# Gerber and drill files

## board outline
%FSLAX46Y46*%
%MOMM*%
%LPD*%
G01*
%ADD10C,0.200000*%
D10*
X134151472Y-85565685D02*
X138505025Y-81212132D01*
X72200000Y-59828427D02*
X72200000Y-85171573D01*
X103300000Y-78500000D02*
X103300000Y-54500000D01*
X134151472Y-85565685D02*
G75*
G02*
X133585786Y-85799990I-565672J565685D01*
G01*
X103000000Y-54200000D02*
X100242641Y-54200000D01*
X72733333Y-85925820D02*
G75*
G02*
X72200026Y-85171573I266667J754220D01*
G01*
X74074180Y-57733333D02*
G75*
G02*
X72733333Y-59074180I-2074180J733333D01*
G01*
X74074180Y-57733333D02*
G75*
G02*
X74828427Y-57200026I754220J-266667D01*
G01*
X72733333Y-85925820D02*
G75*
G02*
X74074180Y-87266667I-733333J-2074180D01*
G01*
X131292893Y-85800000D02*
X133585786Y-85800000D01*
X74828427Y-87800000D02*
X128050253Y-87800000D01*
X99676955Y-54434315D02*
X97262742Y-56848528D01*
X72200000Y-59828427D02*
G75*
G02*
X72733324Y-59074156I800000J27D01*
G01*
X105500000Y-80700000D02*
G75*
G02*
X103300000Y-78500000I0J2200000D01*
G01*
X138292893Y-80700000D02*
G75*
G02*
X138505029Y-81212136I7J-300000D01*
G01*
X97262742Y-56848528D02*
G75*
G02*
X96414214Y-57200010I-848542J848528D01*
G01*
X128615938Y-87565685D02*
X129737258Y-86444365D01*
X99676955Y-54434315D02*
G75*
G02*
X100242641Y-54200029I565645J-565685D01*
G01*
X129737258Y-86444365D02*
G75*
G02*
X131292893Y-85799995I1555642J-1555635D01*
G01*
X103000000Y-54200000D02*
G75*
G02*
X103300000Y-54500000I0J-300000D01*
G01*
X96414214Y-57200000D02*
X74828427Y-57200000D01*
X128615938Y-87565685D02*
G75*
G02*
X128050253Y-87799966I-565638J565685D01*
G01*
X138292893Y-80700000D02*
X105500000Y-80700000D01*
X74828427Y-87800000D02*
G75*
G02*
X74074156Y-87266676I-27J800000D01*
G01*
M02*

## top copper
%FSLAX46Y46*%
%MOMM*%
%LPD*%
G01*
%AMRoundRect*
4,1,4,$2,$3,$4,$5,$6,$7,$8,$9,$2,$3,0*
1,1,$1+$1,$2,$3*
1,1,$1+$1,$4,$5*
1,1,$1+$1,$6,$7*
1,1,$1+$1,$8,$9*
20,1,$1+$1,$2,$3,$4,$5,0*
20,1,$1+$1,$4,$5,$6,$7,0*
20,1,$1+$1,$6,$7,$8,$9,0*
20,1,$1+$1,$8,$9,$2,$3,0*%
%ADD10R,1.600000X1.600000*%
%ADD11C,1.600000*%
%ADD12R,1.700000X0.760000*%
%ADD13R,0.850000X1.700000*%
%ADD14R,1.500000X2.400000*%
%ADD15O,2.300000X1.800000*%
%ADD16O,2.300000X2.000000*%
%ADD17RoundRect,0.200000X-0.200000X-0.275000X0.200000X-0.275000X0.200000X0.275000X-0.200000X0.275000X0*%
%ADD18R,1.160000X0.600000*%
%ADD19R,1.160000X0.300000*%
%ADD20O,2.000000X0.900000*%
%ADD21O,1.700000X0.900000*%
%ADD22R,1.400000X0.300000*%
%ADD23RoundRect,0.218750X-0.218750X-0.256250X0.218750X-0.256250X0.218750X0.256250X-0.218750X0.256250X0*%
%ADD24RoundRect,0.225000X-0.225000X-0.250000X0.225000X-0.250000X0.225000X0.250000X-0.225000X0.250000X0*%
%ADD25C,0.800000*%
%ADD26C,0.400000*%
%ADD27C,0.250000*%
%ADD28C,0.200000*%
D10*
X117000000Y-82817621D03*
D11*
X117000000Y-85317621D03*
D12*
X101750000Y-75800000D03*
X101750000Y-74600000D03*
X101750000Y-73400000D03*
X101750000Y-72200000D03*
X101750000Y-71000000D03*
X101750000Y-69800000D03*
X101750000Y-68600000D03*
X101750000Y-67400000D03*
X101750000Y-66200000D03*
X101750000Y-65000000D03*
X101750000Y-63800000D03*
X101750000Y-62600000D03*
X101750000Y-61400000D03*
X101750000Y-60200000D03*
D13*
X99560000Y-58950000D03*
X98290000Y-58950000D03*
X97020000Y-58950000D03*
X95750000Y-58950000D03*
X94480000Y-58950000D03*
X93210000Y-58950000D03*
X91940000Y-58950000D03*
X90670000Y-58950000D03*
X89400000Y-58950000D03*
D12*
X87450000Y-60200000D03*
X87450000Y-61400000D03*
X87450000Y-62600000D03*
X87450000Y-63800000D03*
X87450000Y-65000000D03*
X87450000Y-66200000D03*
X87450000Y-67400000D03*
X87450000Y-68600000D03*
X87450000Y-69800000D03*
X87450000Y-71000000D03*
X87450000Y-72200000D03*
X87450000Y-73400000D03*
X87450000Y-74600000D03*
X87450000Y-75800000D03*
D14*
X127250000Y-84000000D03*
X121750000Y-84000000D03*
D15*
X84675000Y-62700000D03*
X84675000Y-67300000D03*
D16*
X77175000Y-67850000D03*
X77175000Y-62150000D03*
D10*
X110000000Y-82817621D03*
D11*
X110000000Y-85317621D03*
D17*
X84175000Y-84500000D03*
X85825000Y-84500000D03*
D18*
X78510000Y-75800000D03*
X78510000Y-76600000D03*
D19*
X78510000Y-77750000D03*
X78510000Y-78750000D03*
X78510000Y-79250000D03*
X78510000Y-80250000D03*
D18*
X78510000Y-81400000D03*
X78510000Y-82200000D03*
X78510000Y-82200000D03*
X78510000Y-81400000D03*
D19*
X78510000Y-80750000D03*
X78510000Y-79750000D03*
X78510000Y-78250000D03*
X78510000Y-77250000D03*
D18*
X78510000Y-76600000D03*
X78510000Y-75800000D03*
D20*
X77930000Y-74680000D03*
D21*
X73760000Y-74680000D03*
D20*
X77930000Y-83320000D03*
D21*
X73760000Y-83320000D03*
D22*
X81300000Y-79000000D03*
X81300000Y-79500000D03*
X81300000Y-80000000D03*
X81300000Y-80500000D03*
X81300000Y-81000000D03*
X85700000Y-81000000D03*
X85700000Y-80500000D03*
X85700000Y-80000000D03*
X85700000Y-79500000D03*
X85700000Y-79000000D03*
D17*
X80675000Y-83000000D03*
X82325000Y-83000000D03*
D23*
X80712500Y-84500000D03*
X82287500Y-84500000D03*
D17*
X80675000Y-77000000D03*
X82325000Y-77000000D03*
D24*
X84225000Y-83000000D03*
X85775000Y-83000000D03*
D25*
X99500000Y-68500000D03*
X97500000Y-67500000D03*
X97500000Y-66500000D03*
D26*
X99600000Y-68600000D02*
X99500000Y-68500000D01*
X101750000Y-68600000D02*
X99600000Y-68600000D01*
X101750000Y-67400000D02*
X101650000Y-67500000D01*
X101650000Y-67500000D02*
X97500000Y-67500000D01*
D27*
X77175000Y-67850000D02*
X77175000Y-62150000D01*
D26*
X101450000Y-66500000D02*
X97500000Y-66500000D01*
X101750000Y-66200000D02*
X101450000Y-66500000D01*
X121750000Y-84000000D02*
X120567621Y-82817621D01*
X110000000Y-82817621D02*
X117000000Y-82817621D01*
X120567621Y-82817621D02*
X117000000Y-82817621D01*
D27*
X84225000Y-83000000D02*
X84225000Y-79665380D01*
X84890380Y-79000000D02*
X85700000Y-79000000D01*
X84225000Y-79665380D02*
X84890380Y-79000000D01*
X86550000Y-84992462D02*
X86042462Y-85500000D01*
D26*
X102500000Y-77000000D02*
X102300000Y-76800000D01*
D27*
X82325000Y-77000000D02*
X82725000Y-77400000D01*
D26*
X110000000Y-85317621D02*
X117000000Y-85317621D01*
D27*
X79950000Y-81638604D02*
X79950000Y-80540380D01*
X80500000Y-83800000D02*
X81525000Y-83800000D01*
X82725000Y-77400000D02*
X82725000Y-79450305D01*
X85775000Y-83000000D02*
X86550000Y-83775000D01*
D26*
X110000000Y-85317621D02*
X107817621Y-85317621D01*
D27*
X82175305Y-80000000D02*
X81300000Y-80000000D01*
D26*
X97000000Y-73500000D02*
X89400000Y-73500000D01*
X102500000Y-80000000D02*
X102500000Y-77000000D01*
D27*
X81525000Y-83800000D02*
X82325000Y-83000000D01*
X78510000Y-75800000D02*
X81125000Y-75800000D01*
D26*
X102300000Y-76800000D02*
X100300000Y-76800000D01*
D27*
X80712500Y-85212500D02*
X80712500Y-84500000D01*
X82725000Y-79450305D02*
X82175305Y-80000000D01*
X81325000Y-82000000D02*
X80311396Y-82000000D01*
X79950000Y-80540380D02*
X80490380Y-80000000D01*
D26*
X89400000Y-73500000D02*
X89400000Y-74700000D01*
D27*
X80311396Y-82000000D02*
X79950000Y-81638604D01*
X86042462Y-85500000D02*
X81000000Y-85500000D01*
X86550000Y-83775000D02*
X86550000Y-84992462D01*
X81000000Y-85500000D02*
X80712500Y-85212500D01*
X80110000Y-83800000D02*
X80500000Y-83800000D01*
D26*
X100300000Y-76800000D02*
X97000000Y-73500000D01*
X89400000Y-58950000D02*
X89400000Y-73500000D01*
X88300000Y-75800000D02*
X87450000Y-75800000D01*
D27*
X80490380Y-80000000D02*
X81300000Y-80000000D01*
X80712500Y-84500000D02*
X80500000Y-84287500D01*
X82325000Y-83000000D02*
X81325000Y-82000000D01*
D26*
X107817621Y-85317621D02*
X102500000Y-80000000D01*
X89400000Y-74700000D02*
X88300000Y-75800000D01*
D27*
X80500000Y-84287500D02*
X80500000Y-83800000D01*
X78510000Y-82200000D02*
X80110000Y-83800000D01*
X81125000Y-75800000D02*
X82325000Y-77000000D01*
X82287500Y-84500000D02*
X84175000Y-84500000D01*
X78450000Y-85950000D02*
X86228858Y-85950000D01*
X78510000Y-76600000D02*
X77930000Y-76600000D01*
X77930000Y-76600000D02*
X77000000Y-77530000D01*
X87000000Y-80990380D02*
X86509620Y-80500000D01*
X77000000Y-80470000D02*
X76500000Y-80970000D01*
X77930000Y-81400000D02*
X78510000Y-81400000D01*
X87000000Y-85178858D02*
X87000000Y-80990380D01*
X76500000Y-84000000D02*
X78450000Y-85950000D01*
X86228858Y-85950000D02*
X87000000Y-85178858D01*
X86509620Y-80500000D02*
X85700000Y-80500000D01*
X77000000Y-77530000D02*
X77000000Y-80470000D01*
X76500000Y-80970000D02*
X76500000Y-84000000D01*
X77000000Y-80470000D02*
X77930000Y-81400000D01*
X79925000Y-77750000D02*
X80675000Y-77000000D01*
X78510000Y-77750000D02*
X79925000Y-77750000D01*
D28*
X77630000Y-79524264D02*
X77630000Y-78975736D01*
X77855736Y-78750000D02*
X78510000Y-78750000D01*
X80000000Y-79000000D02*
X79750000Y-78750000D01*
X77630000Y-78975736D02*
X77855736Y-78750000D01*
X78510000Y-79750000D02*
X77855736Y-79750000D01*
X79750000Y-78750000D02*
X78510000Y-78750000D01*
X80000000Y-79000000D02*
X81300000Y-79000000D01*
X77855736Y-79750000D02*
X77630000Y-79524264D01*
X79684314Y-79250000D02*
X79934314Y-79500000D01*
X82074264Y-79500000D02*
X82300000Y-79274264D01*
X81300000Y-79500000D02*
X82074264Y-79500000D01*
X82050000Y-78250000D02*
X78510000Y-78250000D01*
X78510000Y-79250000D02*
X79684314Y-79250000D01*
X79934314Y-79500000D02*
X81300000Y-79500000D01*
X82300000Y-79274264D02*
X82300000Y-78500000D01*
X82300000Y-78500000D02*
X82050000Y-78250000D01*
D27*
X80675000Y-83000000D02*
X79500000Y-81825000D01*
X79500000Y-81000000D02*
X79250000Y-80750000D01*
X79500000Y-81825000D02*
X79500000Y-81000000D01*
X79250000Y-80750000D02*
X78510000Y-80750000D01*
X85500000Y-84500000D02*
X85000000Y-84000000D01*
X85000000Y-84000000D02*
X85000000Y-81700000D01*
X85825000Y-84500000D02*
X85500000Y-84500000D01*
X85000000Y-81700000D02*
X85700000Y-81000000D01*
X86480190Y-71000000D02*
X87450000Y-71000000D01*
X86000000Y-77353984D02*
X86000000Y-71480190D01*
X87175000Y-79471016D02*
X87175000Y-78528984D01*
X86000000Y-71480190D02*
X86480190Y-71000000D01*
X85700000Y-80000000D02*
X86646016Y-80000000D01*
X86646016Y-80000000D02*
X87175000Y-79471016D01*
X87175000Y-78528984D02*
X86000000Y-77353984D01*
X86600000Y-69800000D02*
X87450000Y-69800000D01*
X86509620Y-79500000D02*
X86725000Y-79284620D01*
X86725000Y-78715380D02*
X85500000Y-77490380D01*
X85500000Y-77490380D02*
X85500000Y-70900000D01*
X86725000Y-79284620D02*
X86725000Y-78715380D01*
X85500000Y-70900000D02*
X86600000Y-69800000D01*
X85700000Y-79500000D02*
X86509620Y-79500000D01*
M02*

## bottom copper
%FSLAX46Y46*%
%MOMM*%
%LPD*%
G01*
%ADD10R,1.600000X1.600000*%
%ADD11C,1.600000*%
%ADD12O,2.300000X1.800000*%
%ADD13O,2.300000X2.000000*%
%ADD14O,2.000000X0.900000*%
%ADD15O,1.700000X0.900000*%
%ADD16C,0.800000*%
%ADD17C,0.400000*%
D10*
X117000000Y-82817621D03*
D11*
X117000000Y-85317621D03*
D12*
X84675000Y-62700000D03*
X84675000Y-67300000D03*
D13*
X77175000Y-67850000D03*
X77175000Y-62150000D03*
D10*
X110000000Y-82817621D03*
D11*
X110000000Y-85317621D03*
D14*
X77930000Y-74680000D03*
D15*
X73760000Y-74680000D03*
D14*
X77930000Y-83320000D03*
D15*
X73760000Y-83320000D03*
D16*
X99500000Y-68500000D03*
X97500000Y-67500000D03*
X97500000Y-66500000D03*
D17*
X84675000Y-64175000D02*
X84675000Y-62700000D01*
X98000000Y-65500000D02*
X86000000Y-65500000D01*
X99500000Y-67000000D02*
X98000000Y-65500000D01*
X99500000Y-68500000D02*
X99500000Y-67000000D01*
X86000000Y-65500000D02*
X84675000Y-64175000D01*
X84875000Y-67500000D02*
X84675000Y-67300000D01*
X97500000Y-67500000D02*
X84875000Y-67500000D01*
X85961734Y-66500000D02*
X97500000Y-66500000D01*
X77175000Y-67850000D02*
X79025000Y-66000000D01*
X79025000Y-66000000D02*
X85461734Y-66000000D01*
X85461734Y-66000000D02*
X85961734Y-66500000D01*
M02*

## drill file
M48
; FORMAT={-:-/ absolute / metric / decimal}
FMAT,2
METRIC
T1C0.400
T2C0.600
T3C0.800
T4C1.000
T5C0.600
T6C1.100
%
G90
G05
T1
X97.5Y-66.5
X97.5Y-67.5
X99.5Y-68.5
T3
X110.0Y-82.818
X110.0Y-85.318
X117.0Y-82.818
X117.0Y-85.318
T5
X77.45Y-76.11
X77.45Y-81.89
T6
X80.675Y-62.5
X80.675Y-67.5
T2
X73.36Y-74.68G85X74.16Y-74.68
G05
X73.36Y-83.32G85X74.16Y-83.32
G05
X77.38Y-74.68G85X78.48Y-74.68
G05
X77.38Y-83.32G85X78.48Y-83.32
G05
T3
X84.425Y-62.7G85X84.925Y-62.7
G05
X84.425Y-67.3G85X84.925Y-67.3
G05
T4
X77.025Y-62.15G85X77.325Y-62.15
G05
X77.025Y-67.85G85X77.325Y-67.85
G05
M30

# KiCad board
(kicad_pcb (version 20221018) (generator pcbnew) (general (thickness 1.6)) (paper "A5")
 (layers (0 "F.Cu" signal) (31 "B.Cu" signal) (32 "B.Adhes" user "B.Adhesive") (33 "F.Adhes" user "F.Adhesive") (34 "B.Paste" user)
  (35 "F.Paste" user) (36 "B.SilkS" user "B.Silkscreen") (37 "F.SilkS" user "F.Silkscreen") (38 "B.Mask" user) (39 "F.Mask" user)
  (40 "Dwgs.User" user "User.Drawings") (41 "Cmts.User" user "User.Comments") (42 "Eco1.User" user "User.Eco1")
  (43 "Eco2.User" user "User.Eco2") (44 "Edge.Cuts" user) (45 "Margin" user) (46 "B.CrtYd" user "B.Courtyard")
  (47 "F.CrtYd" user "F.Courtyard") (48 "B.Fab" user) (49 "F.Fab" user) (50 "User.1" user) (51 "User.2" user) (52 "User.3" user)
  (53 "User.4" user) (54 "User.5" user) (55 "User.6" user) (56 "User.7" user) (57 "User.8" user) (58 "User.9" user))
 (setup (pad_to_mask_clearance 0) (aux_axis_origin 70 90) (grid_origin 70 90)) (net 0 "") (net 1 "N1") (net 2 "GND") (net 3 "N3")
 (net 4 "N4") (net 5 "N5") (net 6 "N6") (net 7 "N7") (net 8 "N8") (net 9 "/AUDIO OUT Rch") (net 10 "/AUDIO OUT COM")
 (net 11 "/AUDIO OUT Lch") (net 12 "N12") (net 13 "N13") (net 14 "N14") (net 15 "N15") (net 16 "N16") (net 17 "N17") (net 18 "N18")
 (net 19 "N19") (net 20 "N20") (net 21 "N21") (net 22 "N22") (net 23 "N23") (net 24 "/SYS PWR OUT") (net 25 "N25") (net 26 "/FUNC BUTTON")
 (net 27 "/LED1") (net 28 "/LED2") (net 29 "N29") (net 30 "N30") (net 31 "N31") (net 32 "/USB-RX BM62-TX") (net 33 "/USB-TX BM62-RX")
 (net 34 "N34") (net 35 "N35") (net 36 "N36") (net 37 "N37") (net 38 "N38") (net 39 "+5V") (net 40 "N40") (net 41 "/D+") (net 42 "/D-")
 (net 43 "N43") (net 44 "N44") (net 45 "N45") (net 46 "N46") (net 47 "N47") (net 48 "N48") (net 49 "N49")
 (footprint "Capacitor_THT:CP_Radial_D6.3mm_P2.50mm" (layer "F.Cu") (at 117 82.817621 -90)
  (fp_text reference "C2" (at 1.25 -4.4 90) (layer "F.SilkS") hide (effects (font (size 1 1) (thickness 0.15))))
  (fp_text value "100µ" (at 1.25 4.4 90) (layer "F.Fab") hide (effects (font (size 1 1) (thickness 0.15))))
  (pad "1" thru_hole rect (at 0 0 270) (size 1.6 1.6) (drill 0.8) (layers "*.Cu" "*.Mask") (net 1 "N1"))
  (pad "2" thru_hole circle (at 2.5 0 270) (size 1.6 1.6) (drill 0.8) (layers "*.Cu" "*.Mask") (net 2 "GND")))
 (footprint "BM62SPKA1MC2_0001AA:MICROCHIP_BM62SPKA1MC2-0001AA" (layer "F.Cu") (at 102.1 58.6 180)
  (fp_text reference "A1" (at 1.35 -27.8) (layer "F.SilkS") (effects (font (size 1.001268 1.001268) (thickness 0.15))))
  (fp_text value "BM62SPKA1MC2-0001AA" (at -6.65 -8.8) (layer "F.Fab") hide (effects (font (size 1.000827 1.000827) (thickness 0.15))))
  (pad "1" smd rect (at 0.35 -17.2 180) (size 1.7 0.76) (layers "F.Cu" "F.Paste" "F.Mask") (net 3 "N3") (solder_mask_margin 0.102))
  (pad "2" smd rect (at 0.35 -16 180) (size 1.7 0.76) (layers "F.Cu" "F.Paste" "F.Mask") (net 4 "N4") (solder_mask_margin 0.102))
  (pad "3" smd rect (at 0.35 -14.8 180) (size 1.7 0.76) (layers "F.Cu" "F.Paste" "F.Mask") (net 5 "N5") (solder_mask_margin 0.102))
  (pad "4" smd rect (at 0.35 -13.6 180) (size 1.7 0.76) (layers "F.Cu" "F.Paste" "F.Mask") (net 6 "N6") (solder_mask_margin 0.102))
  (pad "5" smd rect (at 0.35 -12.4 180) (size 1.7 0.76) (layers "F.Cu" "F.Paste" "F.Mask") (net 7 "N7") (solder_mask_margin 0.102))
  (pad "6" smd rect (at 0.35 -11.2 180) (size 1.7 0.76) (layers "F.Cu" "F.Paste" "F.Mask") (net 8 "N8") (solder_mask_margin 0.102))
  (pad "7" smd rect (at 0.35 -10 180) (size 1.7 0.76) (layers "F.Cu" "F.Paste" "F.Mask") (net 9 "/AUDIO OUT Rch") (solder_mask_margin 0.102))
  (pad "8" smd rect (at 0.35 -8.8 180) (size 1.7 0.76) (layers "F.Cu" "F.Paste" "F.Mask") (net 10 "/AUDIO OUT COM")
   (solder_mask_margin 0.102))
  (pad "9" smd rect (at 0.35 -7.6 180) (size 1.7 0.76) (layers "F.Cu" "F.Paste" "F.Mask") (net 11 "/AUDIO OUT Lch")
   (solder_mask_margin 0.102))
  (pad "10" smd rect (at 0.35 -6.4 180) (size 1.7 0.76) (layers "F.Cu" "F.Paste" "F.Mask") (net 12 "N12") (solder_mask_margin 0.102))
  (pad "11" smd rect (at 0.35 -5.2 180) (size 1.7 0.76) (layers "F.Cu" "F.Paste" "F.Mask") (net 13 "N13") (solder_mask_margin 0.102))
  (pad "12" smd rect (at 0.35 -4 180) (size 1.7 0.76) (layers "F.Cu" "F.Paste" "F.Mask") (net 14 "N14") (solder_mask_margin 0.102))
  (pad "13" smd rect (at 0.35 -2.8 180) (size 1.7 0.76) (layers "F.Cu" "F.Paste" "F.Mask") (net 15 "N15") (solder_mask_margin 0.102))
  (pad "14" smd rect (at 0.35 -1.6 180) (size 1.7 0.76) (layers "F.Cu" "F.Paste" "F.Mask") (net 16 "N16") (solder_mask_margin 0.102))
  (pad "15" smd rect (at 2.54 -0.35 90) (size 1.7 0.85) (layers "F.Cu" "F.Paste" "F.Mask") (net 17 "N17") (solder_mask_margin 0.102))
  (pad "16" smd rect (at 3.81 -0.35 90) (size 1.7 0.85) (layers "F.Cu" "F.Paste" "F.Mask") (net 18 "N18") (solder_mask_margin 0.102))
  (pad "17" smd rect (at 5.08 -0.35 90) (size 1.7 0.85) (layers "F.Cu" "F.Paste" "F.Mask") (solder_mask_margin 0.102))
  (pad "18" smd rect (at 6.35 -0.35 90) (size 1.7 0.85) (layers "F.Cu" "F.Paste" "F.Mask") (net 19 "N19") (solder_mask_margin 0.102))
  (pad "19" smd rect (at 7.62 -0.35 90) (size 1.7 0.85) (layers "F.Cu" "F.Paste" "F.Mask") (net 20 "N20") (solder_mask_margin 0.102))
  (pad "20" smd rect (at 8.89 -0.35 90) (size 1.7 0.85) (layers "F.Cu" "F.Paste" "F.Mask") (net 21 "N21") (solder_mask_margin 0.102))
  (pad "21" smd rect (at 10.16 -0.35 90) (size 1.7 0.85) (layers "F.Cu" "F.Paste" "F.Mask") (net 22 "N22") (solder_mask_margin 0.102))
  (pad "22" smd rect (at 11.43 -0.35 90) (size 1.7 0.85) (layers "F.Cu" "F.Paste" "F.Mask") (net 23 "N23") (solder_mask_margin 0.102))
  (pad "23" smd rect (at 12.7 -0.35 90) (size 1.7 0.85) (layers "F.Cu" "F.Paste" "F.Mask") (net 2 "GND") (solder_mask_margin 0.102))
  (pad "24" smd rect (at 14.65 -1.6) (size 1.7 0.76) (layers "F.Cu" "F.Paste" "F.Mask") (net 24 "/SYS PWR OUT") (solder_mask_margin 0.102))
  (pad "25" smd rect (at 14.65 -2.8) (size 1.7 0.76) (layers "F.Cu" "F.Paste" "F.Mask") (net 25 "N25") (solder_mask_margin 0.102))
  (pad "26" smd rect (at 14.65 -4) (size 1.7 0.76) (layers "F.Cu" "F.Paste" "F.Mask") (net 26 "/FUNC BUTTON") (solder_mask_margin 0.102))
  (pad "27" smd rect (at 14.65 -5.2) (size 1.7 0.76) (layers "F.Cu" "F.Paste" "F.Mask") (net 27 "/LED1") (solder_mask_margin 0.102))
  (pad "28" smd rect (at 14.65 -6.4) (size 1.7 0.76) (layers "F.Cu" "F.Paste" "F.Mask") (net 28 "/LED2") (solder_mask_margin 0.102))
  (pad "29" smd rect (at 14.65 -7.6) (size 1.7 0.76) (layers "F.Cu" "F.Paste" "F.Mask") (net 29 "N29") (solder_mask_margin 0.102))
  (pad "30" smd rect (at 14.65 -8.8) (size 1.7 0.76) (layers "F.Cu" "F.Paste" "F.Mask") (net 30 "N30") (solder_mask_margin 0.102))
  (pad "31" smd rect (at 14.65 -10) (size 1.7 0.76) (layers "F.Cu" "F.Paste" "F.Mask") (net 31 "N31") (solder_mask_margin 0.102))
  (pad "32" smd rect (at 14.65 -11.2) (size 1.7 0.76) (layers "F.Cu" "F.Paste" "F.Mask") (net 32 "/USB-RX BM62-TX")
   (solder_mask_margin 0.102))
  (pad "33" smd rect (at 14.65 -12.4) (size 1.7 0.76) (layers "F.Cu" "F.Paste" "F.Mask") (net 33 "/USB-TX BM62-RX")
   (solder_mask_margin 0.102))
  (pad "34" smd rect (at 14.65 -13.6) (size 1.7 0.76) (layers "F.Cu" "F.Paste" "F.Mask") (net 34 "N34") (solder_mask_margin 0.102))
  (pad "35" smd rect (at 14.65 -14.8) (size 1.7 0.76) (layers "F.Cu" "F.Paste" "F.Mask") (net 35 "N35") (solder_mask_margin 0.102))
  (pad "36" smd rect (at 14.65 -16) (size 1.7 0.76) (layers "F.Cu" "F.Paste" "F.Mask") (solder_mask_margin 0.102))
  (pad "37" smd rect (at 14.65 -17.2) (size 1.7 0.76) (layers "F.Cu" "F.Paste" "F.Mask") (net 2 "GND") (solder_mask_margin 0.102))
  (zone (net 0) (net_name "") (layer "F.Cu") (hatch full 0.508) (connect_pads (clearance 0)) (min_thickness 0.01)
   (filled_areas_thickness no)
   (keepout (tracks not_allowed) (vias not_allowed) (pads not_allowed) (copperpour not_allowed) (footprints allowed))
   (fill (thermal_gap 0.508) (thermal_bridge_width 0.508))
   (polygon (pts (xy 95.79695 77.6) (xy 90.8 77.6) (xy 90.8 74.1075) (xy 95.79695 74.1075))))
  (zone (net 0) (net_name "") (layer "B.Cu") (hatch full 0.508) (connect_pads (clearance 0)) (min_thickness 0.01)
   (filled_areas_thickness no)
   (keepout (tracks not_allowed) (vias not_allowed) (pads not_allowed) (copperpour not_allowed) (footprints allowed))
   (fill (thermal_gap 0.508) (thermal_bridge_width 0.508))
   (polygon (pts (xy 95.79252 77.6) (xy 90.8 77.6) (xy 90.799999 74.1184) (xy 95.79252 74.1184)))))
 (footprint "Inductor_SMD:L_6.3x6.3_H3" (layer "F.Cu") (at 124.5 84 180)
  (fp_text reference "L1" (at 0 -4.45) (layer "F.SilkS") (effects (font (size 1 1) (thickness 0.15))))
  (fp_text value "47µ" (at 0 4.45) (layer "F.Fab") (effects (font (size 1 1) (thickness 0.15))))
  (pad "1" smd rect (at -2.75 0 180) (size 1.5 2.4) (layers "F.Cu" "F.Paste" "F.Mask") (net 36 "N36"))
  (pad "2" smd rect (at 2.75 0 180) (size 1.5 2.4) (layers "F.Cu" "F.Paste" "F.Mask") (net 1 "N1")))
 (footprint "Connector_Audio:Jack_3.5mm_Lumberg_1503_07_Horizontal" (layer "F.Cu") (at 77.175 67.85 90)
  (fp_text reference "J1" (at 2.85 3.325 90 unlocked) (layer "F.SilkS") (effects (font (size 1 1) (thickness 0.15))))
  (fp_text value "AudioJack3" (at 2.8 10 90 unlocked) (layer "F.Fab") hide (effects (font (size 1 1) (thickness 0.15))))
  (pad "" np_thru_hole circle (at 0.35 3.5 90) (size 1.1 1.1) (drill 1.1) (layers "F&B.Cu" "*.Mask"))
  (pad "" np_thru_hole circle (at 5.35 3.5 90) (size 1.1 1.1) (drill 1.1) (layers "F&B.Cu" "*.Mask"))
  (pad "R" thru_hole oval (at 5.15 7.5 90) (size 1.8 2.3) (drill oval 0.8 1.3) (layers "*.Cu" "*.Mask") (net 9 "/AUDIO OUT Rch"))
  (pad "S" thru_hole oval (at 0.55 7.5 90) (size 1.8 2.3) (drill oval 0.8 1.3) (layers "*.Cu" "*.Mask") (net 10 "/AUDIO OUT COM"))
  (pad "T" thru_hole oval (at 0 0 90) (size 2 2.3) (drill oval 1 1.3) (layers "*.Cu" "*.Mask") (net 11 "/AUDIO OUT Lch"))
  (pad "T" thru_hole oval (at 5.7 0 90) (size 2 2.3) (drill oval 1 1.3) (layers "*.Cu" "*.Mask") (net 11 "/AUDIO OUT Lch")))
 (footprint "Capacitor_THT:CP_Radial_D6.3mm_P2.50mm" (layer "F.Cu") (at 110 82.817621 -90)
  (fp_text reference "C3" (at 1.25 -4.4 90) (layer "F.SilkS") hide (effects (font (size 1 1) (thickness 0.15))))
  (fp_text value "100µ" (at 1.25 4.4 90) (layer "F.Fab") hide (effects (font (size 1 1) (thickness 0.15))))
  (pad "1" thru_hole rect (at 0 0 270) (size 1.6 1.6) (drill 0.8) (layers "*.Cu" "*.Mask") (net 1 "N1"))
  (pad "2" thru_hole circle (at 2.5 0 270) (size 1.6 1.6) (drill 0.8) (layers "*.Cu" "*.Mask") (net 2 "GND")))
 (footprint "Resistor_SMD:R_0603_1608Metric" (layer "F.Cu") (at 85 84.5)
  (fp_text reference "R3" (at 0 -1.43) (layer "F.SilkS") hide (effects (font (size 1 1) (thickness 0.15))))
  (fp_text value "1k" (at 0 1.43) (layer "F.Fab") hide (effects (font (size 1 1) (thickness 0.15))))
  (pad "1" smd roundrect (at -0.825 0) (size 0.8 0.95) (layers "F.Cu" "F.Paste" "F.Mask") (roundrect_rratio 0.25) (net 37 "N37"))
  (pad "2" smd roundrect (at 0.825 0) (size 0.8 0.95) (layers "F.Cu" "F.Paste" "F.Mask") (roundrect_rratio 0.25) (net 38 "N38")))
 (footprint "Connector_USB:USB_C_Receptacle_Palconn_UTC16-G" (layer "F.Cu") (at 76 79 -90)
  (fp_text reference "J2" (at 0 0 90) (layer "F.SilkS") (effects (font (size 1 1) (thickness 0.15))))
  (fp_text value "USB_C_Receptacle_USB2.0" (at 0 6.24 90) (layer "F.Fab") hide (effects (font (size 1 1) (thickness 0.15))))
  (pad "" np_thru_hole circle (at -2.89 -1.45 90) (size 0.6 0.6) (drill 0.6) (layers "*.Cu" "*.Mask"))
  (pad "" np_thru_hole circle (at 2.89 -1.45 90) (size 0.6 0.6) (drill 0.6) (layers "*.Cu" "*.Mask"))
  (pad "A1" smd rect (at -3.2 -2.51 270) (size 0.6 1.16) (layers "F.Cu" "F.Paste" "F.Mask") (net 2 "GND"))
  (pad "A4" smd rect (at -2.4 -2.51 270) (size 0.6 1.16) (layers "F.Cu" "F.Paste" "F.Mask") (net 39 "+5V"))
  (pad "A5" smd rect (at -1.25 -2.51 90) (size 0.3 1.16) (layers "F.Cu" "F.Paste" "F.Mask") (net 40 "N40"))
  (pad "A6" smd rect (at -0.25 -2.51 90) (size 0.3 1.16) (layers "F.Cu" "F.Paste" "F.Mask") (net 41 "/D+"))
  (pad "A7" smd rect (at 0.25 -2.51 90) (size 0.3 1.16) (layers "F.Cu" "F.Paste" "F.Mask") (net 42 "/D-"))
  (pad "A8" smd rect (at 1.25 -2.51 90) (size 0.3 1.16) (layers "F.Cu" "F.Paste" "F.Mask") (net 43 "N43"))
  (pad "A9" smd rect (at 2.4 -2.51 270) (size 0.6 1.16) (layers "F.Cu" "F.Paste" "F.Mask") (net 39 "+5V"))
  (pad "A12" smd rect (at 3.2 -2.51 270) (size 0.6 1.16) (layers "F.Cu" "F.Paste" "F.Mask") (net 2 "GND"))
  (pad "B1" smd rect (at 3.2 -2.51 270) (size 0.6 1.16) (layers "F.Cu" "F.Paste" "F.Mask") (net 2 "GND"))
  (pad "B4" smd rect (at 2.4 -2.51 270) (size 0.6 1.16) (layers "F.Cu" "F.Paste" "F.Mask") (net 39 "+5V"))
  (pad "B5" smd rect (at 1.75 -2.51 90) (size 0.3 1.16) (layers "F.Cu" "F.Paste" "F.Mask") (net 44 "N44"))
  (pad "B6" smd rect (at 0.75 -2.51 90) (size 0.3 1.16) (layers "F.Cu" "F.Paste" "F.Mask") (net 41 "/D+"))
  (pad "B7" smd rect (at -0.75 -2.51 90) (size 0.3 1.16) (layers "F.Cu" "F.Paste" "F.Mask") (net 42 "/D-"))
  (pad "B8" smd rect (at -1.75 -2.51 90) (size 0.3 1.16) (layers "F.Cu" "F.Paste" "F.Mask") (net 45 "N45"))
  (pad "B9" smd rect (at -2.4 -2.51 270) (size 0.6 1.16) (layers "F.Cu" "F.Paste" "F.Mask") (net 39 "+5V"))
  (pad "B12" smd rect (at -3.2 -2.51 270) (size 0.6 1.16) (layers "F.Cu" "F.Paste" "F.Mask") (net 2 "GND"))
  (pad "S1" thru_hole oval (at -4.32 -1.93) (size 2 0.9) (drill oval 1.7 0.6) (layers "*.Cu" "*.Mask") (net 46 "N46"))
  (pad "S1" thru_hole oval (at -4.32 2.24) (size 1.7 0.9) (drill oval 1.4 0.6) (layers "*.Cu" "*.Mask") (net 46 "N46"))
  (pad "S1" thru_hole oval (at 4.32 -1.93) (size 2 0.9) (drill oval 1.7 0.6) (layers "*.Cu" "*.Mask") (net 46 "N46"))
  (pad "S1" thru_hole oval (at 4.32 2.24) (size 1.7 0.9) (drill oval 1.4 0.6) (layers "*.Cu" "*.Mask") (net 46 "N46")))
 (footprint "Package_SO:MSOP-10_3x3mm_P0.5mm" (layer "F.Cu") (at 83.5 80)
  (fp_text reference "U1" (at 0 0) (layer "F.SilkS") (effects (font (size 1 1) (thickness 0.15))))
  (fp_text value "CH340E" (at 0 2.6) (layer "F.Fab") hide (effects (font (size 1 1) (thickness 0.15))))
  (pad "1" smd rect (at -2.2 -1) (size 1.4 0.3) (layers "F.Cu" "F.Paste" "F.Mask") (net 41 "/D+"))
  (pad "2" smd rect (at -2.2 -0.5) (size 1.4 0.3) (layers "F.Cu" "F.Paste" "F.Mask") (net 42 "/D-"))
  (pad "3" smd rect (at -2.2 0) (size 1.4 0.3) (layers "F.Cu" "F.Paste" "F.Mask") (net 2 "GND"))
  (pad "4" smd rect (at -2.2 0.5) (size 1.4 0.3) (layers "F.Cu" "F.Paste" "F.Mask") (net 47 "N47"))
  (pad "5" smd rect (at -2.2 1) (size 1.4 0.3) (layers "F.Cu" "F.Paste" "F.Mask") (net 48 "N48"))
  (pad "6" smd rect (at 2.2 1) (size 1.4 0.3) (layers "F.Cu" "F.Paste" "F.Mask") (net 38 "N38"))
  (pad "7" smd rect (at 2.2 0.5) (size 1.4 0.3) (layers "F.Cu" "F.Paste" "F.Mask") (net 39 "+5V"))
  (pad "8" smd rect (at 2.2 0) (size 1.4 0.3) (layers "F.Cu" "F.Paste" "F.Mask") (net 33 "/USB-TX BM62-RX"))
  (pad "9" smd rect (at 2.2 -0.5) (size 1.4 0.3) (layers "F.Cu" "F.Paste" "F.Mask") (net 32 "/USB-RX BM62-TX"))
  (pad "10" smd rect (at 2.2 -1) (size 1.4 0.3) (layers "F.Cu" "F.Paste" "F.Mask") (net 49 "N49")))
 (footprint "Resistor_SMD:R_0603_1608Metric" (layer "F.Cu") (at 81.5 83)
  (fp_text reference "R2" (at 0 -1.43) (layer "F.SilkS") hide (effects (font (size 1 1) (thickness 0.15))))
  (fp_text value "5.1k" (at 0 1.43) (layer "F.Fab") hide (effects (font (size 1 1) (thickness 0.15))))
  (pad "1" smd roundrect (at -0.825 0) (size 0.8 0.95) (layers "F.Cu" "F.Paste" "F.Mask") (roundrect_rratio 0.25) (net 44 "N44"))
  (pad "2" smd roundrect (at 0.825 0) (size 0.8 0.95) (layers "F.Cu" "F.Paste" "F.Mask") (roundrect_rratio 0.25) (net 2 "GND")))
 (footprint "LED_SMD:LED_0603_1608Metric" (layer "F.Cu") (at 81.5 84.5)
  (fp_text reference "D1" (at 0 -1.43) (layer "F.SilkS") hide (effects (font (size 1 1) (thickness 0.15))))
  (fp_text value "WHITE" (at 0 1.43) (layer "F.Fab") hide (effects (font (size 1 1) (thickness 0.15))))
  (pad "1" smd roundrect (at -0.7875 0) (size 0.875 0.95) (layers "F.Cu" "F.Paste" "F.Mask") (roundrect_rratio 0.25) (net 2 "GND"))
  (pad "2" smd roundrect (at 0.7875 0) (size 0.875 0.95) (layers "F.Cu" "F.Paste" "F.Mask") (roundrect_rratio 0.25) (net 37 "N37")))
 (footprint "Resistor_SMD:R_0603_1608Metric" (layer "F.Cu") (at 81.5 77)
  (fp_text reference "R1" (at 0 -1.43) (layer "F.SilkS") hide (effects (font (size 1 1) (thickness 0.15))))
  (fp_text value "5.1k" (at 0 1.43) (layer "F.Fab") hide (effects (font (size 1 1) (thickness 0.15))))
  (pad "1" smd roundrect (at -0.825 0) (size 0.8 0.95) (layers "F.Cu" "F.Paste" "F.Mask") (roundrect_rratio 0.25) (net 40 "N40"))
  (pad "2" smd roundrect (at 0.825 0) (size 0.8 0.95) (layers "F.Cu" "F.Paste" "F.Mask") (roundrect_rratio 0.25) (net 2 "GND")))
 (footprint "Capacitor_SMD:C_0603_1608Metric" (layer "F.Cu") (at 85 83)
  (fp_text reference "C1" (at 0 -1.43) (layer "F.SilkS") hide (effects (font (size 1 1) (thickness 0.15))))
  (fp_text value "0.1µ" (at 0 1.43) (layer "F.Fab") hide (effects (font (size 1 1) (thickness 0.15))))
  (pad "1" smd roundrect (at -0.775 0) (size 0.9 0.95) (layers "F.Cu" "F.Paste" "F.Mask") (roundrect_rratio 0.25) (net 49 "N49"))
  (pad "2" smd roundrect (at 0.775 0) (size 0.9 0.95) (layers "F.Cu" "F.Paste" "F.Mask") (roundrect_rratio 0.25) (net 2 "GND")))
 (gr_line (start 134.151472 85.565685) (end 138.505025 81.212132) (stroke (width 0.2) (type solid)) (layer "Edge.Cuts"))
 (gr_line (start 72.2 59.828427) (end 72.2 85.171573) (stroke (width 0.2) (type solid)) (layer "Edge.Cuts"))
 (gr_line (start 103.3 78.5) (end 103.3 54.5) (stroke (width 0.2) (type solid)) (layer "Edge.Cuts"))
 (gr_arc (start 134.151472 85.565685) (mid 133.891933 85.739104) (end 133.585786 85.8) (stroke (width 0.2) (type solid)) (layer "Edge.Cuts"))
 (gr_line (start 103 54.2) (end 100.242641 54.2) (stroke (width 0.2) (type solid)) (layer "Edge.Cuts"))
 (gr_arc (start 72.733333 85.92582) (mid 72.346803 85.633453) (end 72.2 85.171573) (stroke (width 0.2) (type solid)) (layer "Edge.Cuts"))
 (gr_arc (start 74.07418 57.733333) (mid 73.555635 58.555635) (end 72.733333 59.07418) (stroke (width 0.2) (type solid)) (layer "Edge.Cuts"))
 (gr_arc (start 74.07418 57.733333) (mid 74.366547 57.346803) (end 74.828427 57.2) (stroke (width 0.2) (type solid)) (layer "Edge.Cuts"))
 (gr_arc (start 72.733333 85.92582) (mid 73.555635 86.444365) (end 74.07418 87.266667) (stroke (width 0.2) (type solid)) (layer "Edge.Cuts"))
 (gr_line (start 131.292893 85.8) (end 133.585786 85.8) (stroke (width 0.2) (type solid)) (layer "Edge.Cuts"))
 (gr_line (start 74.828427 87.8) (end 128.050253 87.8) (stroke (width 0.2) (type solid)) (layer "Edge.Cuts"))
 (gr_line (start 99.676955 54.434315) (end 97.262742 56.848528) (stroke (width 0.2) (type solid)) (layer "Edge.Cuts"))
 (gr_arc (start 72.2 59.828427) (mid 72.346803 59.366547) (end 72.733333 59.07418) (stroke (width 0.2) (type solid)) (layer "Edge.Cuts"))
 (gr_arc (start 105.5 80.7) (mid 103.944365 80.055635) (end 103.3 78.5) (stroke (width 0.2) (type solid)) (layer "Edge.Cuts"))
 (gr_arc (start 138.292893 80.7) (mid 138.570057 80.885195) (end 138.505025 81.212132) (stroke (width 0.2) (type solid)) (layer "Edge.Cuts"))
 (gr_arc (start 97.262742 56.848528) (mid 96.873434 57.108655) (end 96.414214 57.2) (stroke (width 0.2) (type solid)) (layer "Edge.Cuts"))
 (gr_line (start 128.615938 87.565685) (end 129.737258 86.444365) (stroke (width 0.2) (type solid)) (layer "Edge.Cuts"))
 (gr_arc (start 99.676955 54.434315) (mid 99.936494 54.260896) (end 100.242641 54.2) (stroke (width 0.2) (type solid)) (layer "Edge.Cuts"))
 (gr_arc (start 129.737258 86.444365) (mid 130.45099 85.967465) (end 131.292893 85.8) (stroke (width 0.2) (type solid)) (layer "Edge.Cuts"))
 (gr_arc (start 103 54.2) (mid 103.212132 54.287868) (end 103.3 54.5) (stroke (width 0.2) (type solid)) (layer "Edge.Cuts"))
 (gr_line (start 96.414214 57.2) (end 74.828427 57.2) (stroke (width 0.2) (type solid)) (layer "Edge.Cuts"))
 (gr_arc (start 128.615938 87.565685) (mid 128.3564 87.739104) (end 128.050253 87.8) (stroke (width 0.2) (type solid)) (layer "Edge.Cuts"))
 (gr_line (start 138.292893 80.7) (end 105.5 80.7) (stroke (width 0.2) (type solid)) (layer "Edge.Cuts"))
 (gr_arc (start 74.828427 87.8) (mid 74.366547 87.653197) (end 74.07418 87.266667) (stroke (width 0.2) (type solid)) (layer "Edge.Cuts"))
 (segment (start 99.6 68.6) (end 99.5 68.5) (width 0.4) (layer "F.Cu") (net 9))
 (segment (start 101.75 68.6) (end 99.6 68.6) (width 0.4) (layer "F.Cu") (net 9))
 (via (at 99.5 68.5) (size 0.8) (drill 0.4) (layers "F.Cu" "B.Cu") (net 9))
 (segment (start 84.675 64.175) (end 84.675 62.7) (width 0.4) (layer "B.Cu") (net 9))
 (segment (start 98 65.5) (end 86 65.5) (width 0.4) (layer "B.Cu") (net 9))
 (segment (start 99.5 67) (end 98 65.5) (width 0.4) (layer "B.Cu") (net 9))
 (segment (start 99.5 68.5) (end 99.5 67) (width 0.4) (layer "B.Cu") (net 9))
 (segment (start 86 65.5) (end 84.675 64.175) (width 0.4) (layer "B.Cu") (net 9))
 (segment (start 101.75 67.4) (end 101.65 67.5) (width 0.4) (layer "F.Cu") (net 10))
 (segment (start 101.65 67.5) (end 97.5 67.5) (width 0.4) (layer "F.Cu") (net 10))
 (via (at 97.5 67.5) (size 0.8) (drill 0.4) (layers "F.Cu" "B.Cu") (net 10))
 (segment (start 84.875 67.5) (end 84.675 67.3) (width 0.4) (layer "B.Cu") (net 10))
 (segment (start 97.5 67.5) (end 84.875 67.5) (width 0.4) (layer "B.Cu") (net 10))
 (segment (start 77.175 67.85) (end 77.175 62.15) (width 0.25) (layer "F.Cu") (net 11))
 (segment (start 101.45 66.5) (end 97.5 66.5) (width 0.4) (layer "F.Cu") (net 11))
 (segment (start 101.75 66.2) (end 101.45 66.5) (width 0.4) (layer "F.Cu") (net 11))
 (via (at 97.5 66.5) (size 0.8) (drill 0.4) (layers "F.Cu" "B.Cu") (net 11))
 (segment (start 85.961734 66.5) (end 97.5 66.5) (width 0.4) (layer "B.Cu") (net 11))
 (segment (start 77.175 67.85) (end 79.025 66) (width 0.4) (layer "B.Cu") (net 11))
 (segment (start 79.025 66) (end 85.461734 66) (width 0.4) (layer "B.Cu") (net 11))
 (segment (start 85.461734 66) (end 85.961734 66.5) (width 0.4) (layer "B.Cu") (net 11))
 (segment (start 121.75 84) (end 120.567621 82.817621) (width 0.4) (layer "F.Cu") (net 1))
 (segment (start 110 82.817621) (end 117 82.817621) (width 0.4) (layer "F.Cu") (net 1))
 (segment (start 120.567621 82.817621) (end 117 82.817621) (width 0.4) (layer "F.Cu") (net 1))
 (segment (start 84.225 83) (end 84.225 79.66538) (width 0.25) (layer "F.Cu") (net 49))
 (segment (start 84.89038 79) (end 85.7 79) (width 0.25) (layer "F.Cu") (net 49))
 (segment (start 84.225 79.66538) (end 84.89038 79) (width 0.25) (layer "F.Cu") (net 49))
 (segment (start 86.55 84.992462) (end 86.042462 85.5) (width 0.25) (layer "F.Cu") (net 2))
 (segment (start 102.5 77) (end 102.3 76.8) (width 0.4) (layer "F.Cu") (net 2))
 (segment (start 82.325 77) (end 82.725 77.4) (width 0.25) (layer "F.Cu") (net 2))
 (segment (start 110 85.317621) (end 117 85.317621) (width 0.4) (layer "F.Cu") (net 2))
 (segment (start 79.95 81.638604) (end 79.95 80.54038) (width 0.25) (layer "F.Cu") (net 2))
 (segment (start 80.5 83.8) (end 81.525 83.8) (width 0.25) (layer "F.Cu") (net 2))
 (segment (start 82.725 77.4) (end 82.725 79.450305) (width 0.25) (layer "F.Cu") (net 2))
 (segment (start 85.775 83) (end 86.55 83.775) (width 0.25) (layer "F.Cu") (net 2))
 (segment (start 110 85.317621) (end 107.817621 85.317621) (width 0.4) (layer "F.Cu") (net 2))
 (segment (start 82.175305 80) (end 81.3 80) (width 0.25) (layer "F.Cu") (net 2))
 (segment (start 97 73.5) (end 89.4 73.5) (width 0.4) (layer "F.Cu") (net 2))
 (segment (start 102.5 80) (end 102.5 77) (width 0.4) (layer "F.Cu") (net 2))
 (segment (start 81.525 83.8) (end 82.325 83) (width 0.25) (layer "F.Cu") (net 2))
 (segment (start 78.51 75.8) (end 81.125 75.8) (width 0.25) (layer "F.Cu") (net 2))
 (segment (start 102.3 76.8) (end 100.3 76.8) (width 0.4) (layer "F.Cu") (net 2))
 (segment (start 80.7125 85.2125) (end 80.7125 84.5) (width 0.25) (layer "F.Cu") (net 2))
 (segment (start 82.725 79.450305) (end 82.175305 80) (width 0.25) (layer "F.Cu") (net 2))
 (segment (start 81.325 82) (end 80.311396 82) (width 0.25) (layer "F.Cu") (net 2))
 (segment (start 79.95 80.54038) (end 80.49038 80) (width 0.25) (layer "F.Cu") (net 2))
 (segment (start 89.4 73.5) (end 89.4 74.7) (width 0.4) (layer "F.Cu") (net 2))
 (segment (start 80.311396 82) (end 79.95 81.638604) (width 0.25) (layer "F.Cu") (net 2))
 (segment (start 86.042462 85.5) (end 81 85.5) (width 0.25) (layer "F.Cu") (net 2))
 (segment (start 86.55 83.775) (end 86.55 84.992462) (width 0.25) (layer "F.Cu") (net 2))
 (segment (start 81 85.5) (end 80.7125 85.2125) (width 0.25) (layer "F.Cu") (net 2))
 (segment (start 80.11 83.8) (end 80.5 83.8) (width 0.25) (layer "F.Cu") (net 2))
 (segment (start 100.3 76.8) (end 97 73.5) (width 0.4) (layer "F.Cu") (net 2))
 (segment (start 89.4 58.95) (end 89.4 73.5) (width 0.4) (layer "F.Cu") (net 2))
 (segment (start 88.3 75.8) (end 87.45 75.8) (width 0.4) (layer "F.Cu") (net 2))
 (segment (start 80.49038 80) (end 81.3 80) (width 0.25) (layer "F.Cu") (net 2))
 (segment (start 80.7125 84.5) (end 80.5 84.2875) (width 0.25) (layer "F.Cu") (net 2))
 (segment (start 82.325 83) (end 81.325 82) (width 0.25) (layer "F.Cu") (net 2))
 (segment (start 107.817621 85.317621) (end 102.5 80) (width 0.4) (layer "F.Cu") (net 2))
 (segment (start 89.4 74.7) (end 88.3 75.8) (width 0.4) (layer "F.Cu") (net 2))
 (segment (start 80.5 84.2875) (end 80.5 83.8) (width 0.25) (layer "F.Cu") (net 2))
 (segment (start 78.51 82.2) (end 80.11 83.8) (width 0.25) (layer "F.Cu") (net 2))
 (segment (start 81.125 75.8) (end 82.325 77) (width 0.25) (layer "F.Cu") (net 2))
 (segment (start 82.2875 84.5) (end 84.175 84.5) (width 0.25) (layer "F.Cu") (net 37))
 (segment (start 78.45 85.95) (end 86.228858 85.95) (width 0.25) (layer "F.Cu") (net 39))
 (segment (start 78.51 76.6) (end 77.93 76.6) (width 0.25) (layer "F.Cu") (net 39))
 (segment (start 77.93 76.6) (end 77 77.53) (width 0.25) (layer "F.Cu") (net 39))
 (segment (start 87 80.99038) (end 86.50962 80.5) (width 0.25) (layer "F.Cu") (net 39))
 (segment (start 77 80.47) (end 76.5 80.97) (width 0.25) (layer "F.Cu") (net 39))
 (segment (start 77.93 81.4) (end 78.51 81.4) (width 0.25) (layer "F.Cu") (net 39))
 (segment (start 87 85.178858) (end 87 80.99038) (width 0.25) (layer "F.Cu") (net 39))
 (segment (start 76.5 84) (end 78.45 85.95) (width 0.25) (layer "F.Cu") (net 39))
 (segment (start 86.228858 85.95) (end 87 85.178858) (width 0.25) (layer "F.Cu") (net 39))
 (segment (start 86.50962 80.5) (end 85.7 80.5) (width 0.25) (layer "F.Cu") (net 39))
 (segment (start 77 77.53) (end 77 80.47) (width 0.25) (layer "F.Cu") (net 39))
 (segment (start 76.5 80.97) (end 76.5 84) (width 0.25) (layer "F.Cu") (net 39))
 (segment (start 77 80.47) (end 77.93 81.4) (width 0.25) (layer "F.Cu") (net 39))
 (segment (start 79.925 77.75) (end 80.675 77) (width 0.25) (layer "F.Cu") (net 40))
 (segment (start 78.51 77.75) (end 79.925 77.75) (width 0.25) (layer "F.Cu") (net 40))
 (segment (start 77.63 79.524264) (end 77.63 78.975736) (width 0.2) (layer "F.Cu") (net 41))
 (segment (start 77.855736 78.75) (end 78.51 78.75) (width 0.2) (layer "F.Cu") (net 41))
 (segment (start 80 79) (end 79.75 78.75) (width 0.2) (layer "F.Cu") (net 41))
 (segment (start 77.63 78.975736) (end 77.855736 78.75) (width 0.2) (layer "F.Cu") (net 41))
 (segment (start 78.51 79.75) (end 77.855736 79.75) (width 0.2) (layer "F.Cu") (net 41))
 (segment (start 79.75 78.75) (end 78.51 78.75) (width 0.2) (layer "F.Cu") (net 41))
 (segment (start 80 79) (end 81.3 79) (width 0.2) (layer "F.Cu") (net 41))
 (segment (start 77.855736 79.75) (end 77.63 79.524264) (width 0.2) (layer "F.Cu") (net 41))
 (segment (start 79.684314 79.25) (end 79.934314 79.5) (width 0.2) (layer "F.Cu") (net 42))
 (segment (start 82.074264 79.5) (end 82.3 79.274264) (width 0.2) (layer "F.Cu") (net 42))
 (segment (start 81.3 79.5) (end 82.074264 79.5) (width 0.2) (layer "F.Cu") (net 42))
 (segment (start 82.05 78.25) (end 78.51 78.25) (width 0.2) (layer "F.Cu") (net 42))
 (segment (start 78.51 79.25) (end 79.684314 79.25) (width 0.2) (layer "F.Cu") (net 42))
 (segment (start 79.934314 79.5) (end 81.3 79.5) (width 0.2) (layer "F.Cu") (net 42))
 (segment (start 82.3 79.274264) (end 82.3 78.5) (width 0.2) (layer "F.Cu") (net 42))
 (segment (start 82.3 78.5) (end 82.05 78.25) (width 0.2) (layer "F.Cu") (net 42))
 (segment (start 80.675 83) (end 79.5 81.825) (width 0.25) (layer "F.Cu") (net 44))
 (segment (start 79.5 81) (end 79.25 80.75) (width 0.25) (layer "F.Cu") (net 44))
 (segment (start 79.5 81.825) (end 79.5 81) (width 0.25) (layer "F.Cu") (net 44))
 (segment (start 79.25 80.75) (end 78.51 80.75) (width 0.25) (layer "F.Cu") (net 44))
 (segment (start 85.5 84.5) (end 85 84) (width 0.25) (layer "F.Cu") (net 38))
 (segment (start 85 84) (end 85 81.7) (width 0.25) (layer "F.Cu") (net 38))
 (segment (start 85.825 84.5) (end 85.5 84.5) (width 0.25) (layer "F.Cu") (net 38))
 (segment (start 85 81.7) (end 85.7 81) (width 0.25) (layer "F.Cu") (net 38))
 (segment (start 86.48019 71) (end 87.45 71) (width 0.25) (layer "F.Cu") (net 33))
 (segment (start 86 77.353984) (end 86 71.48019) (width 0.25) (layer "F.Cu") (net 33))
 (segment (start 87.175 79.471016) (end 87.175 78.528984) (width 0.25) (layer "F.Cu") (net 33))
 (segment (start 86 71.48019) (end 86.48019 71) (width 0.25) (layer "F.Cu") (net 33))
 (segment (start 85.7 80) (end 86.646016 80) (width 0.25) (layer "F.Cu") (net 33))
 (segment (start 86.646016 80) (end 87.175 79.471016) (width 0.25) (layer "F.Cu") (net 33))
 (segment (start 87.175 78.528984) (end 86 77.353984) (width 0.25) (layer "F.Cu") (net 33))
 (segment (start 86.6 69.8) (end 87.45 69.8) (width 0.25) (layer "F.Cu") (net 32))
 (segment (start 86.50962 79.5) (end 86.725 79.28462) (width 0.25) (layer "F.Cu") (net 32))
 (segment (start 86.725 78.71538) (end 85.5 77.49038) (width 0.25) (layer "F.Cu") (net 32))
 (segment (start 85.5 77.49038) (end 85.5 70.9) (width 0.25) (layer "F.Cu") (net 32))
 (segment (start 86.725 79.28462) (end 86.725 78.71538) (width 0.25) (layer "F.Cu") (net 32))
 (segment (start 85.5 70.9) (end 86.6 69.8) (width 0.25) (layer "F.Cu") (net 32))
 (segment (start 85.7 79.5) (end 86.50962 79.5) (width 0.25) (layer "F.Cu") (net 32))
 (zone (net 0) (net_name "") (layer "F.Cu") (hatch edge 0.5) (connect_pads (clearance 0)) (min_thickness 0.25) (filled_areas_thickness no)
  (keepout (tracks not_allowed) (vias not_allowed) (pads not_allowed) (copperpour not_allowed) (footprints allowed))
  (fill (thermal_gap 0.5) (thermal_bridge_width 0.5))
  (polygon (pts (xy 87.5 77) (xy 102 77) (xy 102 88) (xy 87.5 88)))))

